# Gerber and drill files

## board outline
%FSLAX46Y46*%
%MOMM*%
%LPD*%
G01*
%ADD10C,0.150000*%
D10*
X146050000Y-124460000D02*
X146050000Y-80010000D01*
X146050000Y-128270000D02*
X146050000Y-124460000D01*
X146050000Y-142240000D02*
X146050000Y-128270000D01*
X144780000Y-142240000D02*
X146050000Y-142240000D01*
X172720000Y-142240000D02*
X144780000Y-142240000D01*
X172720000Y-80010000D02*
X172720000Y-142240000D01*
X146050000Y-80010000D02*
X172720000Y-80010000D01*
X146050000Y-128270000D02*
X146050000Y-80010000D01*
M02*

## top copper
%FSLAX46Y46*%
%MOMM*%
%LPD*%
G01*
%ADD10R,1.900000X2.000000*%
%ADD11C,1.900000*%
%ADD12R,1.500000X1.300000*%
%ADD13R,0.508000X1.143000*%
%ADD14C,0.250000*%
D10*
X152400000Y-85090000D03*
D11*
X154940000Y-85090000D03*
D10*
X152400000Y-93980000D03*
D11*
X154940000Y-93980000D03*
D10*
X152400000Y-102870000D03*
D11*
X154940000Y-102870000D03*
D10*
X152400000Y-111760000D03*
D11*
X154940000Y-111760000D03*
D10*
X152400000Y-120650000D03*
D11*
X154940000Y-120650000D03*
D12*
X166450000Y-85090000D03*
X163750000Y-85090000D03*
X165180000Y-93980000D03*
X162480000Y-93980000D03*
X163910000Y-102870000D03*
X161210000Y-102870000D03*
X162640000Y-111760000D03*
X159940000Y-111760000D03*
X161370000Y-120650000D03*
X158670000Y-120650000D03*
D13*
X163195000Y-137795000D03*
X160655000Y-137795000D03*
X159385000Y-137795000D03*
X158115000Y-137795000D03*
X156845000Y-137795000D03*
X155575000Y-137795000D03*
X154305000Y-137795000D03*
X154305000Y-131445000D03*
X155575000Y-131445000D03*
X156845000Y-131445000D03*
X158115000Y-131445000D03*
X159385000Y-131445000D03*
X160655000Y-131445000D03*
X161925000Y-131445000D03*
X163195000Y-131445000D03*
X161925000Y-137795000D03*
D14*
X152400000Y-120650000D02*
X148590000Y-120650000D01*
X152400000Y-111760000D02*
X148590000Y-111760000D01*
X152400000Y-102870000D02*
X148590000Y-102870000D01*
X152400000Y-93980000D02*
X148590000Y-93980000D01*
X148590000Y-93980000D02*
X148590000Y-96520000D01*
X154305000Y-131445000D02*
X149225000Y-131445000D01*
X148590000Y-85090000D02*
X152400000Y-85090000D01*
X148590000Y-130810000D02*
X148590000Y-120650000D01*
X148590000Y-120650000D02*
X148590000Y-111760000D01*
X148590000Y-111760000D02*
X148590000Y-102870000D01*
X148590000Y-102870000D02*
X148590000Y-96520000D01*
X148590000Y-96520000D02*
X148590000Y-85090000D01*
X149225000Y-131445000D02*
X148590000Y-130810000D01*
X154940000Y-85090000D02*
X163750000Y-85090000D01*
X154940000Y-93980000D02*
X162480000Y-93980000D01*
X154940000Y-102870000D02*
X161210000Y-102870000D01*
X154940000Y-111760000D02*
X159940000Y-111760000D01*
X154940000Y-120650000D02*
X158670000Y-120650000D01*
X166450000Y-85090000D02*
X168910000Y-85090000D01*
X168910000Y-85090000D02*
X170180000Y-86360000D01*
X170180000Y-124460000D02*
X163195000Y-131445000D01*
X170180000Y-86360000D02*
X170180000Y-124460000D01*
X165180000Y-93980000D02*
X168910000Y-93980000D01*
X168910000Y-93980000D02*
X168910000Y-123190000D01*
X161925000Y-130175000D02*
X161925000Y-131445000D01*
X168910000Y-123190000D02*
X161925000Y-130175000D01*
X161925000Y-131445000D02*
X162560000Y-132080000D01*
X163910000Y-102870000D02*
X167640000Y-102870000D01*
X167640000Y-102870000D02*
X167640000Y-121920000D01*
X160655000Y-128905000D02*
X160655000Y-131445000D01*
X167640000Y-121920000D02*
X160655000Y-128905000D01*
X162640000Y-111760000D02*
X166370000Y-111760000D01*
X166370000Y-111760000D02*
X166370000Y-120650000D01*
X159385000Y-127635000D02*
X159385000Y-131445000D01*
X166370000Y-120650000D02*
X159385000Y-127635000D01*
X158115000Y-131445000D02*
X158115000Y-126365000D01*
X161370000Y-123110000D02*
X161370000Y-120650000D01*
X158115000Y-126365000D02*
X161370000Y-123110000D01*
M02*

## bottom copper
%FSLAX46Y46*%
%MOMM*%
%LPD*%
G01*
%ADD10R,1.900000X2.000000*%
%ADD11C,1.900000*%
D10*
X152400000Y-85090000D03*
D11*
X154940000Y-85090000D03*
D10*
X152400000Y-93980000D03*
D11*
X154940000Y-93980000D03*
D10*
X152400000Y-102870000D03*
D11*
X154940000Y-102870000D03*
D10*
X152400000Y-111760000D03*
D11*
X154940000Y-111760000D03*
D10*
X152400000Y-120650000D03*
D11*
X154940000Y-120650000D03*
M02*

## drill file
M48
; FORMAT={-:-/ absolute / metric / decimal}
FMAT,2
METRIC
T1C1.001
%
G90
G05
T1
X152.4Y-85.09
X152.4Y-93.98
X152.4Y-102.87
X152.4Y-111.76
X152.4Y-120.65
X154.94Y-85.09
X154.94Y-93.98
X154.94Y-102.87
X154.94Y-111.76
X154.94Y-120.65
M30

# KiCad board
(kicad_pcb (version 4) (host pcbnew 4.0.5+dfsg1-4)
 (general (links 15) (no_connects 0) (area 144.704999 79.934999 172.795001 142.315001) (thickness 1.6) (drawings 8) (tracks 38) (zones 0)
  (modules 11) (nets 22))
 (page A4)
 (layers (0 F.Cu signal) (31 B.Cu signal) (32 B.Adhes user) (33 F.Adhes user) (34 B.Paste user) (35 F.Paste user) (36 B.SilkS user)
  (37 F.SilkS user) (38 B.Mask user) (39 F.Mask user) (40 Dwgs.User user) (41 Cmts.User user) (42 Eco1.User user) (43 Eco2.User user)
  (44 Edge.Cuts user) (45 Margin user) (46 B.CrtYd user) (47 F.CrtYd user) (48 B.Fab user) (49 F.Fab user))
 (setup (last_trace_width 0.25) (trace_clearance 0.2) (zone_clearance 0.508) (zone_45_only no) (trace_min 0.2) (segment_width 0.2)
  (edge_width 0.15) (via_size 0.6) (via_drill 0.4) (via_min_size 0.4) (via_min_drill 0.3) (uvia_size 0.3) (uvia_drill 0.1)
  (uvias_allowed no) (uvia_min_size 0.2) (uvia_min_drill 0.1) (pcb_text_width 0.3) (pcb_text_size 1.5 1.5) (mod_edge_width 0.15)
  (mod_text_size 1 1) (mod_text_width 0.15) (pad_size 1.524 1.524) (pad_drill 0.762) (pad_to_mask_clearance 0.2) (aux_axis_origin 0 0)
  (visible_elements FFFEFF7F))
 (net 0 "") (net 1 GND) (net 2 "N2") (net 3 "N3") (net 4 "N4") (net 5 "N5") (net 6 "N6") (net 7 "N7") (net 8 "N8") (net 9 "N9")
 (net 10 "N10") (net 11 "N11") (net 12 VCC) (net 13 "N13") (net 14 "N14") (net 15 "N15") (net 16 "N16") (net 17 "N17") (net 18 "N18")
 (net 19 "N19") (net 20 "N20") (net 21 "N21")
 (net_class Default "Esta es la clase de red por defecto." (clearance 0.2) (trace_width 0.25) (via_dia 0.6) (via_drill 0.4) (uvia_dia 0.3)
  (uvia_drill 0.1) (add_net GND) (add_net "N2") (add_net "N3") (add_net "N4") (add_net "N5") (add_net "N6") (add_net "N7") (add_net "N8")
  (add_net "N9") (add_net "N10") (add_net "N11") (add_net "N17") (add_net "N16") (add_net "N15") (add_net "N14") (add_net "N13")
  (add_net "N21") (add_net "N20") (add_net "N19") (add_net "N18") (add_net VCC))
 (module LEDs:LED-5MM (layer F.Cu) (at 152.4 85.09)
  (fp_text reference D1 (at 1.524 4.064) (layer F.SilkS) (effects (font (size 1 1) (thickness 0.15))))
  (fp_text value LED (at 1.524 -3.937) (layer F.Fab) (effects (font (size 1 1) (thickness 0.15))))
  (pad 1 thru_hole rect (at 0 0 90) (size 2 1.9) (drill 1.00076) (layers *.Cu *.Mask) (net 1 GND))
  (pad 2 thru_hole circle (at 2.54 0) (size 1.9 1.9) (drill 1.00076) (layers *.Cu *.Mask) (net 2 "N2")))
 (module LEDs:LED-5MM (layer F.Cu) (at 152.4 93.98)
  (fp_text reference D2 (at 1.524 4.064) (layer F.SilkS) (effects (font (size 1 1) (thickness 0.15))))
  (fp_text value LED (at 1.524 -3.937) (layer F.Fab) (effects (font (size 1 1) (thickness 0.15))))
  (pad 1 thru_hole rect (at 0 0 90) (size 2 1.9) (drill 1.00076) (layers *.Cu *.Mask) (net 1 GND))
  (pad 2 thru_hole circle (at 2.54 0) (size 1.9 1.9) (drill 1.00076) (layers *.Cu *.Mask) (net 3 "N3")))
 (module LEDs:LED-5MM (layer F.Cu) (at 152.4 102.87)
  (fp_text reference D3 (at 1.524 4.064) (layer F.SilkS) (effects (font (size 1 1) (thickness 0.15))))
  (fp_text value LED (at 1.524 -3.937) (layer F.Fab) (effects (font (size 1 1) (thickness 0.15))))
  (pad 1 thru_hole rect (at 0 0 90) (size 2 1.9) (drill 1.00076) (layers *.Cu *.Mask) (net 1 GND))
  (pad 2 thru_hole circle (at 2.54 0) (size 1.9 1.9) (drill 1.00076) (layers *.Cu *.Mask) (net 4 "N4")))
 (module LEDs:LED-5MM (layer F.Cu) (at 152.4 111.76)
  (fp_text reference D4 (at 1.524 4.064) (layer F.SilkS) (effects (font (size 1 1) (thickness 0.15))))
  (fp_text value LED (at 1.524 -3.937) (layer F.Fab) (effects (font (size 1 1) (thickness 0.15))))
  (pad 1 thru_hole rect (at 0 0 90) (size 2 1.9) (drill 1.00076) (layers *.Cu *.Mask) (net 1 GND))
  (pad 2 thru_hole circle (at 2.54 0) (size 1.9 1.9) (drill 1.00076) (layers *.Cu *.Mask) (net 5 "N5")))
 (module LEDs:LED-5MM (layer F.Cu) (at 152.4 120.65)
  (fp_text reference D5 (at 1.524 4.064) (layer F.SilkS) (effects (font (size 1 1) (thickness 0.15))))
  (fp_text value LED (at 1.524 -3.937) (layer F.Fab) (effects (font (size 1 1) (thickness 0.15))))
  (pad 1 thru_hole rect (at 0 0 90) (size 2 1.9) (drill 1.00076) (layers *.Cu *.Mask) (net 1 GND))
  (pad 2 thru_hole circle (at 2.54 0) (size 1.9 1.9) (drill 1.00076) (layers *.Cu *.Mask) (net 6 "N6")))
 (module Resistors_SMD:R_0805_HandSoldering (layer F.Cu) (at 165.1 85.09 180)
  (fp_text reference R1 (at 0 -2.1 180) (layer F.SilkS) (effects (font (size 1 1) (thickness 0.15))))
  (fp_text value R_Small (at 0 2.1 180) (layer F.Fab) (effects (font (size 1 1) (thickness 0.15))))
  (pad 1 smd rect (at -1.35 0 180) (size 1.5 1.3) (layers F.Cu F.Paste F.Mask) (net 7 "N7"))
  (pad 2 smd rect (at 1.35 0 180) (size 1.5 1.3) (layers F.Cu F.Paste F.Mask) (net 2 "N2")))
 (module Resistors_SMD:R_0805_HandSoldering (layer F.Cu) (at 163.83 93.98 180)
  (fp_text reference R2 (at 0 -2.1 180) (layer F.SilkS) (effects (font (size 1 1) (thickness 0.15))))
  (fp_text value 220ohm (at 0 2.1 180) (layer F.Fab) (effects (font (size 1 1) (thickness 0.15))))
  (pad 1 smd rect (at -1.35 0 180) (size 1.5 1.3) (layers F.Cu F.Paste F.Mask) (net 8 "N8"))
  (pad 2 smd rect (at 1.35 0 180) (size 1.5 1.3) (layers F.Cu F.Paste F.Mask) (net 3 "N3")))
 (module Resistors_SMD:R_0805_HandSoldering (layer F.Cu) (at 162.56 102.87 180)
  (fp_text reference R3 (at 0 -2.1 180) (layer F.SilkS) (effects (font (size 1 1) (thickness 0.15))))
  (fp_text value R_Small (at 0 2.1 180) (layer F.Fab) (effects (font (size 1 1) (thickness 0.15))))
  (pad 1 smd rect (at -1.35 0 180) (size 1.5 1.3) (layers F.Cu F.Paste F.Mask) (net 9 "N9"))
  (pad 2 smd rect (at 1.35 0 180) (size 1.5 1.3) (layers F.Cu F.Paste F.Mask) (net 4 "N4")))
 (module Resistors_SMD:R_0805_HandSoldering (layer F.Cu) (at 161.29 111.76 180)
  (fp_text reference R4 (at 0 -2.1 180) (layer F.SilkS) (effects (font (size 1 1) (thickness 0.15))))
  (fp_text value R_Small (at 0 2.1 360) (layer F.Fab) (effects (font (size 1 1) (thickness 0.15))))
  (pad 1 smd rect (at -1.35 0 180) (size 1.5 1.3) (layers F.Cu F.Paste F.Mask) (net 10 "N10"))
  (pad 2 smd rect (at 1.35 0 180) (size 1.5 1.3) (layers F.Cu F.Paste F.Mask) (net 5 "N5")))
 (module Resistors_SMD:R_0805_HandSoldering (layer F.Cu) (at 160.02 120.65 180)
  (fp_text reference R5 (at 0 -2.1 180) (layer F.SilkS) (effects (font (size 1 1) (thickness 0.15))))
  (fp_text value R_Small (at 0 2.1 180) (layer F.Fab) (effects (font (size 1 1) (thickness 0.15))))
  (pad 1 smd rect (at -1.35 0 180) (size 1.5 1.3) (layers F.Cu F.Paste F.Mask) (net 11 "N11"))
  (pad 2 smd rect (at 1.35 0 180) (size 1.5 1.3) (layers F.Cu F.Paste F.Mask) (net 6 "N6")))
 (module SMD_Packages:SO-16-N (layer F.Cu) (at 158.75 134.62 180)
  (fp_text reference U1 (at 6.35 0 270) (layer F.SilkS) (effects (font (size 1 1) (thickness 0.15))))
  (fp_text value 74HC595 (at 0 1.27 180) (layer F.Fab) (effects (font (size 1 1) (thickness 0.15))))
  (pad 16 smd rect (at -4.445 -3.175 180) (size 0.508 1.143) (layers F.Cu F.Paste F.Mask) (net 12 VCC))
  (pad 14 smd rect (at -1.905 -3.175 180) (size 0.508 1.143) (layers F.Cu F.Paste F.Mask) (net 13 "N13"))
  (pad 13 smd rect (at -0.635 -3.175 180) (size 0.508 1.143) (layers F.Cu F.Paste F.Mask) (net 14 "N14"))
  (pad 12 smd rect (at 0.635 -3.175 180) (size 0.508 1.143) (layers F.Cu F.Paste F.Mask) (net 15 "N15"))
  (pad 11 smd rect (at 1.905 -3.175 180) (size 0.508 1.143) (layers F.Cu F.Paste F.Mask) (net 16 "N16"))
  (pad 10 smd rect (at 3.175 -3.175 180) (size 0.508 1.143) (layers F.Cu F.Paste F.Mask) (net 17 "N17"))
  (pad 9 smd rect (at 4.445 -3.175 180) (size 0.508 1.143) (layers F.Cu F.Paste F.Mask) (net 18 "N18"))
  (pad 8 smd rect (at 4.445 3.175 180) (size 0.508 1.143) (layers F.Cu F.Paste F.Mask) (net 1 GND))
  (pad 7 smd rect (at 3.175 3.175 180) (size 0.508 1.143) (layers F.Cu F.Paste F.Mask) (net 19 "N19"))
  (pad 6 smd rect (at 1.905 3.175 180) (size 0.508 1.143) (layers F.Cu F.Paste F.Mask) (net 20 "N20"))
  (pad 5 smd rect (at 0.635 3.175 180) (size 0.508 1.143) (layers F.Cu F.Paste F.Mask) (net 11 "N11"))
  (pad 4 smd rect (at -0.635 3.175 180) (size 0.508 1.143) (layers F.Cu F.Paste F.Mask) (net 10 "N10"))
  (pad 3 smd rect (at -1.905 3.175 180) (size 0.508 1.143) (layers F.Cu F.Paste F.Mask) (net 9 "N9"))
  (pad 2 smd rect (at -3.175 3.175 180) (size 0.508 1.143) (layers F.Cu F.Paste F.Mask) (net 8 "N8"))
  (pad 1 smd rect (at -4.445 3.175 180) (size 0.508 1.143) (layers F.Cu F.Paste F.Mask) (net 7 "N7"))
  (pad 15 smd rect (at -3.175 -3.175 180) (size 0.508 1.143) (layers F.Cu F.Paste F.Mask) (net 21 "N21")))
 (gr_line (start 146.05 124.46) (end 146.05 80.01) (angle 90) (layer Edge.Cuts) (width 0.15))
 (gr_line (start 146.05 128.27) (end 146.05 124.46) (angle 90) (layer Edge.Cuts) (width 0.15))
 (gr_line (start 146.05 142.24) (end 146.05 128.27) (angle 90) (layer Edge.Cuts) (width 0.15))
 (gr_line (start 144.78 142.24) (end 146.05 142.24) (angle 90) (layer Edge.Cuts) (width 0.15))
 (gr_line (start 172.72 142.24) (end 144.78 142.24) (angle 90) (layer Edge.Cuts) (width 0.15))
 (gr_line (start 172.72 80.01) (end 172.72 142.24) (angle 90) (layer Edge.Cuts) (width 0.15))
 (gr_line (start 146.05 80.01) (end 172.72 80.01) (angle 90) (layer Edge.Cuts) (width 0.15))
 (gr_line (start 146.05 128.27) (end 146.05 80.01) (angle 90) (layer Edge.Cuts) (width 0.15))
 (segment (start 152.4 120.65) (end 148.59 120.65) (width 0.25) (layer F.Cu) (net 1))
 (segment (start 152.4 111.76) (end 148.59 111.76) (width 0.25) (layer F.Cu) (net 1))
 (segment (start 152.4 102.87) (end 148.59 102.87) (width 0.25) (layer F.Cu) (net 1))
 (segment (start 152.4 93.98) (end 148.59 93.98) (width 0.25) (layer F.Cu) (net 1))
 (segment (start 148.59 93.98) (end 148.59 96.52) (width 0.25) (layer F.Cu) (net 1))
 (segment (start 154.305 131.445) (end 149.225 131.445) (width 0.25) (layer F.Cu) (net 1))
 (segment (start 148.59 85.09) (end 152.4 85.09) (width 0.25) (layer F.Cu) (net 1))
 (segment (start 148.59 130.81) (end 148.59 120.65) (width 0.25) (layer F.Cu) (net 1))
 (segment (start 148.59 120.65) (end 148.59 111.76) (width 0.25) (layer F.Cu) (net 1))
 (segment (start 148.59 111.76) (end 148.59 102.87) (width 0.25) (layer F.Cu) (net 1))
 (segment (start 148.59 102.87) (end 148.59 96.52) (width 0.25) (layer F.Cu) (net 1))
 (segment (start 148.59 96.52) (end 148.59 85.09) (width 0.25) (layer F.Cu) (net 1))
 (segment (start 149.225 131.445) (end 148.59 130.81) (width 0.25) (layer F.Cu) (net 1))
 (segment (start 154.94 85.09) (end 163.75 85.09) (width 0.25) (layer F.Cu) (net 2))
 (segment (start 154.94 93.98) (end 162.48 93.98) (width 0.25) (layer F.Cu) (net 3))
 (segment (start 154.94 102.87) (end 161.21 102.87) (width 0.25) (layer F.Cu) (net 4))
 (segment (start 154.94 111.76) (end 159.94 111.76) (width 0.25) (layer F.Cu) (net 5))
 (segment (start 154.94 120.65) (end 158.67 120.65) (width 0.25) (layer F.Cu) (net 6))
 (segment (start 166.45 85.09) (end 168.91 85.09) (width 0.25) (layer F.Cu) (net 7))
 (segment (start 168.91 85.09) (end 170.18 86.36) (width 0.25) (layer F.Cu) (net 7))
 (segment (start 170.18 124.46) (end 163.195 131.445) (width 0.25) (layer F.Cu) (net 7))
 (segment (start 170.18 86.36) (end 170.18 124.46) (width 0.25) (layer F.Cu) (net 7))
 (segment (start 165.18 93.98) (end 168.91 93.98) (width 0.25) (layer F.Cu) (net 8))
 (segment (start 168.91 93.98) (end 168.91 123.19) (width 0.25) (layer F.Cu) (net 8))
 (segment (start 161.925 130.175) (end 161.925 131.445) (width 0.25) (layer F.Cu) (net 8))
 (segment (start 168.91 123.19) (end 161.925 130.175) (width 0.25) (layer F.Cu) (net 8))
 (segment (start 161.925 131.445) (end 162.56 132.08) (width 0.25) (layer F.Cu) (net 8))
 (segment (start 163.91 102.87) (end 167.64 102.87) (width 0.25) (layer F.Cu) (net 9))
 (segment (start 167.64 102.87) (end 167.64 121.92) (width 0.25) (layer F.Cu) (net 9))
 (segment (start 160.655 128.905) (end 160.655 131.445) (width 0.25) (layer F.Cu) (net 9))
 (segment (start 167.64 121.92) (end 160.655 128.905) (width 0.25) (layer F.Cu) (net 9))
 (segment (start 162.64 111.76) (end 166.37 111.76) (width 0.25) (layer F.Cu) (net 10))
 (segment (start 166.37 111.76) (end 166.37 120.65) (width 0.25) (layer F.Cu) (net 10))
 (segment (start 159.385 127.635) (end 159.385 131.445) (width 0.25) (layer F.Cu) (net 10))
 (segment (start 166.37 120.65) (end 159.385 127.635) (width 0.25) (layer F.Cu) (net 10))
 (segment (start 158.115 131.445) (end 158.115 126.365) (width 0.25) (layer F.Cu) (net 11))
 (segment (start 161.37 123.11) (end 161.37 120.65) (width 0.25) (layer F.Cu) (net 11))
 (segment (start 158.115 126.365) (end 161.37 123.11) (width 0.25) (layer F.Cu) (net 11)))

